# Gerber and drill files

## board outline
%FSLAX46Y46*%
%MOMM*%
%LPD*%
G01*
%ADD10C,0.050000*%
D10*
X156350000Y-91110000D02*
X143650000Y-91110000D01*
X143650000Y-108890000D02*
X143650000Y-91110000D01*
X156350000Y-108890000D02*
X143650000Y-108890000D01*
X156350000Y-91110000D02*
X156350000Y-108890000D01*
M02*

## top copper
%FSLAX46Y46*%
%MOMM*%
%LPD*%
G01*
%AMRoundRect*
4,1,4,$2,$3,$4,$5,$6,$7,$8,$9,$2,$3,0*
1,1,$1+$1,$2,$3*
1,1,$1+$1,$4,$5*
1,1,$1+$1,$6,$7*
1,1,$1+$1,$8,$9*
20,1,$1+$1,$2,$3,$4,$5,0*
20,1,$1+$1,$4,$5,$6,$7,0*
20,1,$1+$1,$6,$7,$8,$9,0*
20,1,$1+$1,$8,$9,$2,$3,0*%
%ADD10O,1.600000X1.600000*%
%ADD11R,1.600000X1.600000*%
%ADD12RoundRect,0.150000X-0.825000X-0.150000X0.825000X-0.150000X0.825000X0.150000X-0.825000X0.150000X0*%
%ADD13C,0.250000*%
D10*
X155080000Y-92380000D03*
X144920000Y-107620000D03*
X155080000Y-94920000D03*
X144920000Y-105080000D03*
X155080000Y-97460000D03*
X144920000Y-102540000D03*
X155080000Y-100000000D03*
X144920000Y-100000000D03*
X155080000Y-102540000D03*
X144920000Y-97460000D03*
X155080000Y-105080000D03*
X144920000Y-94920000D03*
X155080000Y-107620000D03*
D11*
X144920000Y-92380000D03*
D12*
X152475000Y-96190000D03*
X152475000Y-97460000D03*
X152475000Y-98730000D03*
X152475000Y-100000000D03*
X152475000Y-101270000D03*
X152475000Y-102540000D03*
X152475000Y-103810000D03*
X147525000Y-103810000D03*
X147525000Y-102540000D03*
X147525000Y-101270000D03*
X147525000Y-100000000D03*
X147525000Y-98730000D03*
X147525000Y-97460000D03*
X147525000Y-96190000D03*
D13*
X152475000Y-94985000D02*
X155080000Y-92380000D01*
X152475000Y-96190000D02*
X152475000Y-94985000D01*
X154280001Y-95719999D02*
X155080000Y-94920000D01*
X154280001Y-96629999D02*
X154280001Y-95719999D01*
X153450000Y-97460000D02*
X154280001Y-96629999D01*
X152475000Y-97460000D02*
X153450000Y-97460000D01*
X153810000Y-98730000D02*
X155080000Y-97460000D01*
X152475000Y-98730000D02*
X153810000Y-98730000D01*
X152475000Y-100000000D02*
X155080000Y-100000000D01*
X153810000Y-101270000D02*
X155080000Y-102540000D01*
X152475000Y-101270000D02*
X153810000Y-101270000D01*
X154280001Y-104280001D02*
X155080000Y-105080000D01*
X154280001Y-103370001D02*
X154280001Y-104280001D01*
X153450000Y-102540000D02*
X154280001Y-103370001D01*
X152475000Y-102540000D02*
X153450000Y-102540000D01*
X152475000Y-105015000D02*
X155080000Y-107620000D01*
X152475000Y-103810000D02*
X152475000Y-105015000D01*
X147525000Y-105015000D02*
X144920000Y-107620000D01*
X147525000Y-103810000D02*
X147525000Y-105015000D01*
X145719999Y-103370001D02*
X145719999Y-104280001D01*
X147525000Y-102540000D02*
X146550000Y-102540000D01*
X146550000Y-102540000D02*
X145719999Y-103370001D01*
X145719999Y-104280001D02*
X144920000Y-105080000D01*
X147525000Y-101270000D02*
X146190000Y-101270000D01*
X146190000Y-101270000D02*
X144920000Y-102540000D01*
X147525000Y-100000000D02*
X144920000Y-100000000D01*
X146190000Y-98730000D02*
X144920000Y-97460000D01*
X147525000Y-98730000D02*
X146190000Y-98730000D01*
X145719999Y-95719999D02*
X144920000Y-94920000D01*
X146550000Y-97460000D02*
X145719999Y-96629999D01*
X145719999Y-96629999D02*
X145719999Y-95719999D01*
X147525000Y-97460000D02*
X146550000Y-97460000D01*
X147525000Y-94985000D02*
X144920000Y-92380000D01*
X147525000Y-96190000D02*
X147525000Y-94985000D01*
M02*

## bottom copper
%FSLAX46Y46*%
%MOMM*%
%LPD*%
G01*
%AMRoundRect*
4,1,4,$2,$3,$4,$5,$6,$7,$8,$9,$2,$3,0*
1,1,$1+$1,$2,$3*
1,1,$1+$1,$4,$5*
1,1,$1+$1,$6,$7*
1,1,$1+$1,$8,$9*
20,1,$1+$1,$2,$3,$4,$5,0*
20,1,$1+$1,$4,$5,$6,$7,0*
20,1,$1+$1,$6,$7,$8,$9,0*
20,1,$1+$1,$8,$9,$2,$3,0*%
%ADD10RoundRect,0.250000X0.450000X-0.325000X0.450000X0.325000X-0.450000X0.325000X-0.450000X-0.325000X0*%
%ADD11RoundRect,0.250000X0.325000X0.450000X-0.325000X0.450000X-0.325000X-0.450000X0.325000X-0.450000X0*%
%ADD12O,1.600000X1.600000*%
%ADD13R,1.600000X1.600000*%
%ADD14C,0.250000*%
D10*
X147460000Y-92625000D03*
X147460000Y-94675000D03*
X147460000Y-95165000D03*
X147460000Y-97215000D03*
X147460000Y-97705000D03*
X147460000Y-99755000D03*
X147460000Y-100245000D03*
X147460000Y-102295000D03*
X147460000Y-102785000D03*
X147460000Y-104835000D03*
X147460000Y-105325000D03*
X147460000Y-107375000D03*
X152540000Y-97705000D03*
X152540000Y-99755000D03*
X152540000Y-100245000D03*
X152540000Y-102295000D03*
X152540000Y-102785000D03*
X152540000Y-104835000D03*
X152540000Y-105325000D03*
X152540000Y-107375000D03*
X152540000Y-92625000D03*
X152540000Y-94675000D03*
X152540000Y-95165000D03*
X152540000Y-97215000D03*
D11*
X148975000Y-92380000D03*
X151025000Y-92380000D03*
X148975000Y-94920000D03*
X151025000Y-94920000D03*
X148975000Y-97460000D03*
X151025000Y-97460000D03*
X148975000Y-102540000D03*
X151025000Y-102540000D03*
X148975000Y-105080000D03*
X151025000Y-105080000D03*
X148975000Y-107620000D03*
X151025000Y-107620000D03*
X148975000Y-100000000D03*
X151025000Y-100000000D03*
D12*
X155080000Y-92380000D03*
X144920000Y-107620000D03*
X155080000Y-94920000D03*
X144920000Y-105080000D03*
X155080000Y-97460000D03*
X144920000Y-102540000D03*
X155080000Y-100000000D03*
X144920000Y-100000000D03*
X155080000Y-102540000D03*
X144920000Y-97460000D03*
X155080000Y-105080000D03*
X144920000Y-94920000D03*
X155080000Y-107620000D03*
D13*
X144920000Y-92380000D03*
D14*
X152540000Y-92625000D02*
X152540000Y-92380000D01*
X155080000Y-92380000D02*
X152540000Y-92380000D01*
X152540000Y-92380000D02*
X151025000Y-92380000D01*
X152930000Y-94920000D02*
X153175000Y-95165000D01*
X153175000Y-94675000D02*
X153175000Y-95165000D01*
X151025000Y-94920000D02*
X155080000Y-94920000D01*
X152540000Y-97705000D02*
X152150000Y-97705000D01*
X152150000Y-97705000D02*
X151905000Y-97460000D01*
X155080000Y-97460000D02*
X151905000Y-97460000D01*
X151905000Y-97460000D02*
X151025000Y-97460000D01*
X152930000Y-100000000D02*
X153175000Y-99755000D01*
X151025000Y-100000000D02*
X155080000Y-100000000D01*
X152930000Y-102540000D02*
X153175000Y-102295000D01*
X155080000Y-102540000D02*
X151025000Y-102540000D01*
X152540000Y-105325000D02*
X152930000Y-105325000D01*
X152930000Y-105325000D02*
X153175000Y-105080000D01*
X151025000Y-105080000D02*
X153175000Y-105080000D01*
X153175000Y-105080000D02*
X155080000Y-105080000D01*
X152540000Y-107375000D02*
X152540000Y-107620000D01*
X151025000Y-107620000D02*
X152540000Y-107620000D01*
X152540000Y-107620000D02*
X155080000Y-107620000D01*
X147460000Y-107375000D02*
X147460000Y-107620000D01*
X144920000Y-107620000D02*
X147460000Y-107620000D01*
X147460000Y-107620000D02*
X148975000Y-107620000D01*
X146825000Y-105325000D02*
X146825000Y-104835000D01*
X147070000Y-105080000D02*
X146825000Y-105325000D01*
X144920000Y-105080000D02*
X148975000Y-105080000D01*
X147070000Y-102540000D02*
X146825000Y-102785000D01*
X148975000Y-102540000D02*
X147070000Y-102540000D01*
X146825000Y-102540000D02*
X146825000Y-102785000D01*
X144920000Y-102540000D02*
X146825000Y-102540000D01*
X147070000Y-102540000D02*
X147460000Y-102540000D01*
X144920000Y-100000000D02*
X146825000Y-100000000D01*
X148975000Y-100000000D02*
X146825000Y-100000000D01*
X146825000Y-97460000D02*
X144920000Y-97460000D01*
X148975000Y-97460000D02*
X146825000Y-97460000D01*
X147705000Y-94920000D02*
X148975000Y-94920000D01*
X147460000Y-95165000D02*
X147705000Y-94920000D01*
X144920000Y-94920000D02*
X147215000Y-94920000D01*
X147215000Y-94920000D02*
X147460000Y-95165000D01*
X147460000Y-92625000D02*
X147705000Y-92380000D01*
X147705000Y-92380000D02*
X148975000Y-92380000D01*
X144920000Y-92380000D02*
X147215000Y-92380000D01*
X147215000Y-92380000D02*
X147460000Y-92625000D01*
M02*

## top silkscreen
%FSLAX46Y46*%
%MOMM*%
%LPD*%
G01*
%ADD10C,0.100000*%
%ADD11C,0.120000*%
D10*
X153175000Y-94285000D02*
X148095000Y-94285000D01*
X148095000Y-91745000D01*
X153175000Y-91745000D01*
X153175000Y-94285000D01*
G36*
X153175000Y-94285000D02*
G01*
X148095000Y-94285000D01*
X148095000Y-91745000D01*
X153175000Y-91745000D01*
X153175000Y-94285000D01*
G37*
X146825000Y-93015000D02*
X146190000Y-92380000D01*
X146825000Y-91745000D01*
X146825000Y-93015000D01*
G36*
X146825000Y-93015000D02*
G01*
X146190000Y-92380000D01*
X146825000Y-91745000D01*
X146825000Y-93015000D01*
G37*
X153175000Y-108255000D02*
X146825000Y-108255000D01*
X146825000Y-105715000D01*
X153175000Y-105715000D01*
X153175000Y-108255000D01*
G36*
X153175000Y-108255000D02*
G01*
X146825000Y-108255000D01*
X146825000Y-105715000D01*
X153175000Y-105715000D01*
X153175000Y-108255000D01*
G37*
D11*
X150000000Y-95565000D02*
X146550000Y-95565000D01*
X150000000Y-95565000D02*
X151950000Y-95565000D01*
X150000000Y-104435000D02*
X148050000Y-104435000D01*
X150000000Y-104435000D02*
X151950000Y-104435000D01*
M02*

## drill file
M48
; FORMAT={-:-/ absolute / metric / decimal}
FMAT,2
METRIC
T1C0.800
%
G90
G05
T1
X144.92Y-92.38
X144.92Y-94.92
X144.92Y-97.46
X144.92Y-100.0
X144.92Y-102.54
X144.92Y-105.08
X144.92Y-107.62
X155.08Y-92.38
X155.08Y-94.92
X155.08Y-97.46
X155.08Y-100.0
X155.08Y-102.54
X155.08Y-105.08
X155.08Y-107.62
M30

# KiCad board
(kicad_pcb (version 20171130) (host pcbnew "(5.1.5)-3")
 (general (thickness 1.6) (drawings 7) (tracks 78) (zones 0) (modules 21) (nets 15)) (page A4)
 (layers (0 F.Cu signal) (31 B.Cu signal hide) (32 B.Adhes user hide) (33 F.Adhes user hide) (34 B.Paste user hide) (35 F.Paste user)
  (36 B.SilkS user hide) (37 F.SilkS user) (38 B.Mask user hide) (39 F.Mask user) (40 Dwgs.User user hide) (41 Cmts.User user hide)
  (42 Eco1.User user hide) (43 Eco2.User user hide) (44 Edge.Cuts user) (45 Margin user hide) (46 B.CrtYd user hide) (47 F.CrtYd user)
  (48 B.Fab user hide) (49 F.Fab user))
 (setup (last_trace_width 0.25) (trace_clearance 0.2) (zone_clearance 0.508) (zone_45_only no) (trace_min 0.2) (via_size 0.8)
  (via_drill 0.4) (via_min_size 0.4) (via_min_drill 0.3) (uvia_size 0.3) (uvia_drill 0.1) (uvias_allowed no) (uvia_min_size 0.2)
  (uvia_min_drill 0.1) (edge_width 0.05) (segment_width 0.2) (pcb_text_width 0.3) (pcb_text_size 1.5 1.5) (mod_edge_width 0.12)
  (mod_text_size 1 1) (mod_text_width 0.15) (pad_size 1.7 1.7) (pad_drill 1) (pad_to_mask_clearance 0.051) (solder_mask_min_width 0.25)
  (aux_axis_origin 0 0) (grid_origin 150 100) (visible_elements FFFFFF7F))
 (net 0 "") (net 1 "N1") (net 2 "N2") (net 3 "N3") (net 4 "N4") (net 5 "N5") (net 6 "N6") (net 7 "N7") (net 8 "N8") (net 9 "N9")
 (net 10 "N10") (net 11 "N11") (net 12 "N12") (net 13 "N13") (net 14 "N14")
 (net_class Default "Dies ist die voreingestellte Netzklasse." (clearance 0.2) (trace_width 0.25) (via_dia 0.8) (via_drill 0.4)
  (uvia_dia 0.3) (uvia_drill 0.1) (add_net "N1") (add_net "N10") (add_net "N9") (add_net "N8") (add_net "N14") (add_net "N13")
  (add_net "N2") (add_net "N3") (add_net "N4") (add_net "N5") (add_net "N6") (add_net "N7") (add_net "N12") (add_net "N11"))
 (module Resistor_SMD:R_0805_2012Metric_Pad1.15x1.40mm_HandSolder (layer B.Cu) (at 147.46 93.65 90)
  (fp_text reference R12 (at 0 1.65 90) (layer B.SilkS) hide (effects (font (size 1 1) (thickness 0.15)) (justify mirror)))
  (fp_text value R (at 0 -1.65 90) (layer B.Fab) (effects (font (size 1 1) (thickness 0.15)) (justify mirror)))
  (pad 2 smd roundrect (at 1.025 0 90) (size 1.15 1.4) (layers B.Cu B.Paste B.Mask) (roundrect_rratio 0.217391) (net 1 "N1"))
  (pad 1 smd roundrect (at -1.025 0 90) (size 1.15 1.4) (layers B.Cu B.Paste B.Mask) (roundrect_rratio 0.217391) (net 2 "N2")))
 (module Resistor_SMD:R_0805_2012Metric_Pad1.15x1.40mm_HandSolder (layer B.Cu) (at 147.46 96.19 90)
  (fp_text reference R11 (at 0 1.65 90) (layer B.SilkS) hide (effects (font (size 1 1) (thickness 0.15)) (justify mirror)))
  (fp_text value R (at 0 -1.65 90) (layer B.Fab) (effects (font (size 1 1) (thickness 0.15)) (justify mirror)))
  (pad 2 smd roundrect (at 1.025 0 90) (size 1.15 1.4) (layers B.Cu B.Paste B.Mask) (roundrect_rratio 0.217391) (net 2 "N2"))
  (pad 1 smd roundrect (at -1.025 0 90) (size 1.15 1.4) (layers B.Cu B.Paste B.Mask) (roundrect_rratio 0.217391) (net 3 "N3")))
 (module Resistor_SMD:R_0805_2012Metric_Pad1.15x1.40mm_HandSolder (layer B.Cu) (at 147.46 98.73 90)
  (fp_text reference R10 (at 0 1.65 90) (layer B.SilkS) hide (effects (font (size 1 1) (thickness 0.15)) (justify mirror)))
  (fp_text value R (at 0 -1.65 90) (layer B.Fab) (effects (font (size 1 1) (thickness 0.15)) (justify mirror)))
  (pad 2 smd roundrect (at 1.025 0 90) (size 1.15 1.4) (layers B.Cu B.Paste B.Mask) (roundrect_rratio 0.217391) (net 3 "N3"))
  (pad 1 smd roundrect (at -1.025 0 90) (size 1.15 1.4) (layers B.Cu B.Paste B.Mask) (roundrect_rratio 0.217391) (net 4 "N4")))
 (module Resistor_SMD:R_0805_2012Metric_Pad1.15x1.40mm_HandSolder (layer B.Cu) (at 147.46 101.27 90)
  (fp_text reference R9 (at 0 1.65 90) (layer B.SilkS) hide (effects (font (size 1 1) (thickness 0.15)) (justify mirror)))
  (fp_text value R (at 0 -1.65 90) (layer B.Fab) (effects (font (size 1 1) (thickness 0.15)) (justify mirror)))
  (pad 2 smd roundrect (at 1.025 0 90) (size 1.15 1.4) (layers B.Cu B.Paste B.Mask) (roundrect_rratio 0.217391) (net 4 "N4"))
  (pad 1 smd roundrect (at -1.025 0 90) (size 1.15 1.4) (layers B.Cu B.Paste B.Mask) (roundrect_rratio 0.217391) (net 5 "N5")))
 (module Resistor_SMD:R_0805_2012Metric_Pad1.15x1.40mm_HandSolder (layer B.Cu) (at 147.46 103.81 90)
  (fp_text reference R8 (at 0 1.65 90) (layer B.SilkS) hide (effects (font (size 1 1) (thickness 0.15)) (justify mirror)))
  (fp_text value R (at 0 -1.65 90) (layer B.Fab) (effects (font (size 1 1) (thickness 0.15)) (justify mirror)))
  (pad 2 smd roundrect (at 1.025 0 90) (size 1.15 1.4) (layers B.Cu B.Paste B.Mask) (roundrect_rratio 0.217391) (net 5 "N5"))
  (pad 1 smd roundrect (at -1.025 0 90) (size 1.15 1.4) (layers B.Cu B.Paste B.Mask) (roundrect_rratio 0.217391) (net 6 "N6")))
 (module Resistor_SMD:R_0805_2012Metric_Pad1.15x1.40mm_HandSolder (layer B.Cu) (at 147.46 106.35 90)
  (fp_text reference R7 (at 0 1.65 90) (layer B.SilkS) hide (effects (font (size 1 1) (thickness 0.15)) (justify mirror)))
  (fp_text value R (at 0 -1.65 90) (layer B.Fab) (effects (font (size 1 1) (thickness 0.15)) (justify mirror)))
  (pad 2 smd roundrect (at 1.025 0 90) (size 1.15 1.4) (layers B.Cu B.Paste B.Mask) (roundrect_rratio 0.217391) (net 6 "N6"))
  (pad 1 smd roundrect (at -1.025 0 90) (size 1.15 1.4) (layers B.Cu B.Paste B.Mask) (roundrect_rratio 0.217391) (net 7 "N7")))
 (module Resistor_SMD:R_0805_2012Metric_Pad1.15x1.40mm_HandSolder (layer B.Cu) (at 152.54 98.73 90)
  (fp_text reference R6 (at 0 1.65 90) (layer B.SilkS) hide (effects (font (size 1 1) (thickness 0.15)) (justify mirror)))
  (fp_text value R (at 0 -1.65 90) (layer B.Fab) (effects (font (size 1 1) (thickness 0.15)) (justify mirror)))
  (pad 2 smd roundrect (at 1.025 0 90) (size 1.15 1.4) (layers B.Cu B.Paste B.Mask) (roundrect_rratio 0.217391) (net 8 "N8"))
  (pad 1 smd roundrect (at -1.025 0 90) (size 1.15 1.4) (layers B.Cu B.Paste B.Mask) (roundrect_rratio 0.217391) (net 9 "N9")))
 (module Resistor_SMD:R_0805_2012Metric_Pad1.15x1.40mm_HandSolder (layer B.Cu) (at 152.54 101.27 90)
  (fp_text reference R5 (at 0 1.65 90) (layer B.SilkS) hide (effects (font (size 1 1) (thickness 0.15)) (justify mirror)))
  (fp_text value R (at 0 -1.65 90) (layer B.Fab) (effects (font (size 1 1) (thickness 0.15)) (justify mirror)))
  (pad 2 smd roundrect (at 1.025 0 90) (size 1.15 1.4) (layers B.Cu B.Paste B.Mask) (roundrect_rratio 0.217391) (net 9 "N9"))
  (pad 1 smd roundrect (at -1.025 0 90) (size 1.15 1.4) (layers B.Cu B.Paste B.Mask) (roundrect_rratio 0.217391) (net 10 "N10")))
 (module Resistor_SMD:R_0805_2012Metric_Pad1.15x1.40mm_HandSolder (layer B.Cu) (at 152.54 103.81 90)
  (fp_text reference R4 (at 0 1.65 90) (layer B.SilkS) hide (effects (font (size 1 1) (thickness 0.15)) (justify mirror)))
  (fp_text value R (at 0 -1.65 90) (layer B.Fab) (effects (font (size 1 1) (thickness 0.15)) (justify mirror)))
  (pad 2 smd roundrect (at 1.025 0 90) (size 1.15 1.4) (layers B.Cu B.Paste B.Mask) (roundrect_rratio 0.217391) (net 10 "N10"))
  (pad 1 smd roundrect (at -1.025 0 90) (size 1.15 1.4) (layers B.Cu B.Paste B.Mask) (roundrect_rratio 0.217391) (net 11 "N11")))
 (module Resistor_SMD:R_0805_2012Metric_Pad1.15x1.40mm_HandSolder (layer B.Cu) (at 152.54 106.35 90)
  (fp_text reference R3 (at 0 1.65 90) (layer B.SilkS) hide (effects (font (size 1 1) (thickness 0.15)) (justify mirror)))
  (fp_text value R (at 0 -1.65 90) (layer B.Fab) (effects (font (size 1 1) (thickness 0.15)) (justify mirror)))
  (pad 2 smd roundrect (at 1.025 0 90) (size 1.15 1.4) (layers B.Cu B.Paste B.Mask) (roundrect_rratio 0.217391) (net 11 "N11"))
  (pad 1 smd roundrect (at -1.025 0 90) (size 1.15 1.4) (layers B.Cu B.Paste B.Mask) (roundrect_rratio 0.217391) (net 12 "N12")))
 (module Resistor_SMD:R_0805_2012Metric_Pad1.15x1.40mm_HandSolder (layer B.Cu) (at 152.54 93.65 90)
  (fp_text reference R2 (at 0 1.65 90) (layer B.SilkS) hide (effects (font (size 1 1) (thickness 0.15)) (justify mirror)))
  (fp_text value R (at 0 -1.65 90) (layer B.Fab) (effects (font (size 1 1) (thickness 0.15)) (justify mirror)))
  (pad 2 smd roundrect (at 1.025 0 90) (size 1.15 1.4) (layers B.Cu B.Paste B.Mask) (roundrect_rratio 0.217391) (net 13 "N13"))
  (pad 1 smd roundrect (at -1.025 0 90) (size 1.15 1.4) (layers B.Cu B.Paste B.Mask) (roundrect_rratio 0.217391) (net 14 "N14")))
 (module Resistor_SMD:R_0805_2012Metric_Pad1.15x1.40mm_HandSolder (layer B.Cu) (at 152.54 96.19 90)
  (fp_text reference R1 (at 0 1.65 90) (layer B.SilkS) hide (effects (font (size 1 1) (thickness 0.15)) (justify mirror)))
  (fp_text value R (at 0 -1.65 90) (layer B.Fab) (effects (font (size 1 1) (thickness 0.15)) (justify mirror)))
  (pad 2 smd roundrect (at 1.025 0 90) (size 1.15 1.4) (layers B.Cu B.Paste B.Mask) (roundrect_rratio 0.217391) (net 14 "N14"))
  (pad 1 smd roundrect (at -1.025 0 90) (size 1.15 1.4) (layers B.Cu B.Paste B.Mask) (roundrect_rratio 0.217391) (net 8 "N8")))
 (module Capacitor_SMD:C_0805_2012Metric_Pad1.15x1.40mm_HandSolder (layer B.Cu) (at 150 92.38 180)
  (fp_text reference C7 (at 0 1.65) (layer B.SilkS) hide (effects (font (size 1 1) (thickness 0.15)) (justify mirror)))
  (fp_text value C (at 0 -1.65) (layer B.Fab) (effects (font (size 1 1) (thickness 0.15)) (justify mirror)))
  (pad 2 smd roundrect (at 1.025 0 180) (size 1.15 1.4) (layers B.Cu B.Paste B.Mask) (roundrect_rratio 0.217391) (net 1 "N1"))
  (pad 1 smd roundrect (at -1.025 0 180) (size 1.15 1.4) (layers B.Cu B.Paste B.Mask) (roundrect_rratio 0.217391) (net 13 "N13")))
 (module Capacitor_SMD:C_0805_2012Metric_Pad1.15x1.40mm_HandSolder (layer B.Cu) (at 150 94.92 180)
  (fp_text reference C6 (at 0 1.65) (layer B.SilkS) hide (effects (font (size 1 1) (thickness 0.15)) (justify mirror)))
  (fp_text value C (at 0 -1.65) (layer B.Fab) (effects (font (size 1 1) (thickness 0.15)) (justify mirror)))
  (pad 2 smd roundrect (at 1.025 0 180) (size 1.15 1.4) (layers B.Cu B.Paste B.Mask) (roundrect_rratio 0.217391) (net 2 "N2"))
  (pad 1 smd roundrect (at -1.025 0 180) (size 1.15 1.4) (layers B.Cu B.Paste B.Mask) (roundrect_rratio 0.217391) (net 14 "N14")))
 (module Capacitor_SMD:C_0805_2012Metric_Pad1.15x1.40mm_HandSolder (layer B.Cu) (at 150 97.46 180)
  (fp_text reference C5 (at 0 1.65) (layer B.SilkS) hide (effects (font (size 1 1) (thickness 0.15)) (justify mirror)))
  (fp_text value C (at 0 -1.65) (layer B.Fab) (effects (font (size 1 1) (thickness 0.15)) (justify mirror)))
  (pad 2 smd roundrect (at 1.025 0 180) (size 1.15 1.4) (layers B.Cu B.Paste B.Mask) (roundrect_rratio 0.217391) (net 3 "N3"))
  (pad 1 smd roundrect (at -1.025 0 180) (size 1.15 1.4) (layers B.Cu B.Paste B.Mask) (roundrect_rratio 0.217391) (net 8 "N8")))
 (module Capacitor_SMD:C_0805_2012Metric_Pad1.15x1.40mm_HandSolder (layer B.Cu) (at 150 102.54 180)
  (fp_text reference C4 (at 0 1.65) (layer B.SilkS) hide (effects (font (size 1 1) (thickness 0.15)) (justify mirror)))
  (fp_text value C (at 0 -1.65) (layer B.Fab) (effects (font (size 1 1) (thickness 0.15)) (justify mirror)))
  (pad 2 smd roundrect (at 1.025 0 180) (size 1.15 1.4) (layers B.Cu B.Paste B.Mask) (roundrect_rratio 0.217391) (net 5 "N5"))
  (pad 1 smd roundrect (at -1.025 0 180) (size 1.15 1.4) (layers B.Cu B.Paste B.Mask) (roundrect_rratio 0.217391) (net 10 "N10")))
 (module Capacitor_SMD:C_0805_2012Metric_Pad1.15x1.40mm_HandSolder (layer B.Cu) (at 150 105.08 180)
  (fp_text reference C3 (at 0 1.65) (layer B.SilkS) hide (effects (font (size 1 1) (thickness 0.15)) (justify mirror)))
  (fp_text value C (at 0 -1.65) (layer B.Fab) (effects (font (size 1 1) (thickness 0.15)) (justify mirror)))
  (pad 2 smd roundrect (at 1.025 0 180) (size 1.15 1.4) (layers B.Cu B.Paste B.Mask) (roundrect_rratio 0.217391) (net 6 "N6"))
  (pad 1 smd roundrect (at -1.025 0 180) (size 1.15 1.4) (layers B.Cu B.Paste B.Mask) (roundrect_rratio 0.217391) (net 11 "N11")))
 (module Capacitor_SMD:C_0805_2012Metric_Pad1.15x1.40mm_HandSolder (layer B.Cu) (at 150 107.62 180)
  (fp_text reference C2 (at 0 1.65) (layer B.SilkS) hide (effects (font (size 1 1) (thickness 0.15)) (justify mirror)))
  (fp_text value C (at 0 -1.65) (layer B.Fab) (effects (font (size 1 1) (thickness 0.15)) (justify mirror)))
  (pad 2 smd roundrect (at 1.025 0 180) (size 1.15 1.4) (layers B.Cu B.Paste B.Mask) (roundrect_rratio 0.217391) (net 7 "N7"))
  (pad 1 smd roundrect (at -1.025 0 180) (size 1.15 1.4) (layers B.Cu B.Paste B.Mask) (roundrect_rratio 0.217391) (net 12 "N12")))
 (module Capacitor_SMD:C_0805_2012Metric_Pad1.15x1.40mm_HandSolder (layer B.Cu) (at 150 100 180)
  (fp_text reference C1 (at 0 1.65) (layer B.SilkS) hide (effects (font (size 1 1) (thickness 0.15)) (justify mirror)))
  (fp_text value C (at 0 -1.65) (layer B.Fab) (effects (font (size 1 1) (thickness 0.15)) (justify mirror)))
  (pad 2 smd roundrect (at 1.025 0 180) (size 1.15 1.4) (layers B.Cu B.Paste B.Mask) (roundrect_rratio 0.217391) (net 4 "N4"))
  (pad 1 smd roundrect (at -1.025 0 180) (size 1.15 1.4) (layers B.Cu B.Paste B.Mask) (roundrect_rratio 0.217391) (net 9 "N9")))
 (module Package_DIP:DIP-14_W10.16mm (layer F.Cu) (at 150 100)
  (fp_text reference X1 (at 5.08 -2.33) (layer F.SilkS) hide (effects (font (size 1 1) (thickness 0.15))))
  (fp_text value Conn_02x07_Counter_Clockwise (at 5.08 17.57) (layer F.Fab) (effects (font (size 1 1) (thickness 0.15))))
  (pad 14 thru_hole oval (at 5.08 -7.62) (size 1.6 1.6) (drill 0.8) (layers *.Cu *.Mask) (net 13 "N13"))
  (pad 7 thru_hole oval (at -5.08 7.62) (size 1.6 1.6) (drill 0.8) (layers *.Cu *.Mask) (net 7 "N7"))
  (pad 13 thru_hole oval (at 5.08 -5.08) (size 1.6 1.6) (drill 0.8) (layers *.Cu *.Mask) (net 14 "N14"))
  (pad 6 thru_hole oval (at -5.08 5.08) (size 1.6 1.6) (drill 0.8) (layers *.Cu *.Mask) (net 6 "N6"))
  (pad 12 thru_hole oval (at 5.08 -2.54) (size 1.6 1.6) (drill 0.8) (layers *.Cu *.Mask) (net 8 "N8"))
  (pad 5 thru_hole oval (at -5.08 2.54) (size 1.6 1.6) (drill 0.8) (layers *.Cu *.Mask) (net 5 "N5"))
  (pad 11 thru_hole oval (at 5.08 0) (size 1.6 1.6) (drill 0.8) (layers *.Cu *.Mask) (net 9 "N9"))
  (pad 4 thru_hole oval (at -5.08 0) (size 1.6 1.6) (drill 0.8) (layers *.Cu *.Mask) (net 4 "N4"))
  (pad 10 thru_hole oval (at 5.08 2.54) (size 1.6 1.6) (drill 0.8) (layers *.Cu *.Mask) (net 10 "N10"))
  (pad 3 thru_hole oval (at -5.08 -2.54) (size 1.6 1.6) (drill 0.8) (layers *.Cu *.Mask) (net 3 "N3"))
  (pad 9 thru_hole oval (at 5.08 5.08) (size 1.6 1.6) (drill 0.8) (layers *.Cu *.Mask) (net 11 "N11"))
  (pad 2 thru_hole oval (at -5.08 -5.08) (size 1.6 1.6) (drill 0.8) (layers *.Cu *.Mask) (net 2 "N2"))
  (pad 8 thru_hole oval (at 5.08 7.62) (size 1.6 1.6) (drill 0.8) (layers *.Cu *.Mask) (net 12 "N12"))
  (pad 1 thru_hole rect (at -5.08 -7.62) (size 1.6 1.6) (drill 0.8) (layers *.Cu *.Mask) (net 1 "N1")))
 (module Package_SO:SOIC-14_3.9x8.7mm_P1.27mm (layer F.Cu) (at 150 100)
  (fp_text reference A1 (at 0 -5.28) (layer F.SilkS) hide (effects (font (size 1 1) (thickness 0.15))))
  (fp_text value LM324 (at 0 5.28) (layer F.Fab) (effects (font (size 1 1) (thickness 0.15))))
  (fp_line (start 0 -4.435) (end -3.45 -4.435) (layer F.SilkS) (width 0.12))
  (fp_line (start 0 -4.435) (end 1.95 -4.435) (layer F.SilkS) (width 0.12))
  (fp_line (start 0 4.435) (end -1.95 4.435) (layer F.SilkS) (width 0.12))
  (fp_line (start 0 4.435) (end 1.95 4.435) (layer F.SilkS) (width 0.12))
  (pad 14 smd roundrect (at 2.475 -3.81) (size 1.95 0.6) (layers F.Cu F.Paste F.Mask) (roundrect_rratio 0.25) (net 13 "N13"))
  (pad 13 smd roundrect (at 2.475 -2.54) (size 1.95 0.6) (layers F.Cu F.Paste F.Mask) (roundrect_rratio 0.25) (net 14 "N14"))
  (pad 12 smd roundrect (at 2.475 -1.27) (size 1.95 0.6) (layers F.Cu F.Paste F.Mask) (roundrect_rratio 0.25) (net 8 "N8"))
  (pad 11 smd roundrect (at 2.475 0) (size 1.95 0.6) (layers F.Cu F.Paste F.Mask) (roundrect_rratio 0.25) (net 9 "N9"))
  (pad 10 smd roundrect (at 2.475 1.27) (size 1.95 0.6) (layers F.Cu F.Paste F.Mask) (roundrect_rratio 0.25) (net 10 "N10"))
  (pad 9 smd roundrect (at 2.475 2.54) (size 1.95 0.6) (layers F.Cu F.Paste F.Mask) (roundrect_rratio 0.25) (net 11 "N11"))
  (pad 8 smd roundrect (at 2.475 3.81) (size 1.95 0.6) (layers F.Cu F.Paste F.Mask) (roundrect_rratio 0.25) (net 12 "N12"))
  (pad 7 smd roundrect (at -2.475 3.81) (size 1.95 0.6) (layers F.Cu F.Paste F.Mask) (roundrect_rratio 0.25) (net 7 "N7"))
  (pad 6 smd roundrect (at -2.475 2.54) (size 1.95 0.6) (layers F.Cu F.Paste F.Mask) (roundrect_rratio 0.25) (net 6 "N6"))
  (pad 5 smd roundrect (at -2.475 1.27) (size 1.95 0.6) (layers F.Cu F.Paste F.Mask) (roundrect_rratio 0.25) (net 5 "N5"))
  (pad 4 smd roundrect (at -2.475 0) (size 1.95 0.6) (layers F.Cu F.Paste F.Mask) (roundrect_rratio 0.25) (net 4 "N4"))
  (pad 3 smd roundrect (at -2.475 -1.27) (size 1.95 0.6) (layers F.Cu F.Paste F.Mask) (roundrect_rratio 0.25) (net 3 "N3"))
  (pad 2 smd roundrect (at -2.475 -2.54) (size 1.95 0.6) (layers F.Cu F.Paste F.Mask) (roundrect_rratio 0.25) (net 2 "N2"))
  (pad 1 smd roundrect (at -2.475 -3.81) (size 1.95 0.6) (layers F.Cu F.Paste F.Mask) (roundrect_rratio 0.25) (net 1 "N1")))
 (gr_poly (pts (xy 153.175 94.285) (xy 148.095 94.285) (xy 148.095 91.745) (xy 153.175 91.745)) (layer F.SilkS) (width 0.1))
 (gr_poly (pts (xy 146.825 93.015) (xy 146.19 92.38) (xy 146.825 91.745)) (layer F.SilkS) (width 0.1))
 (gr_poly (pts (xy 153.175 108.255) (xy 146.825 108.255) (xy 146.825 105.715) (xy 153.175 105.715)) (layer F.SilkS) (width 0.1))
 (gr_line (start 156.35 91.11) (end 143.65 91.11) (layer Edge.Cuts) (width 0.05))
 (gr_line (start 143.65 108.89) (end 143.65 91.11) (layer Edge.Cuts) (width 0.05))
 (gr_line (start 156.35 108.89) (end 143.65 108.89) (layer Edge.Cuts) (width 0.05))
 (gr_line (start 156.35 91.11) (end 156.35 108.89) (layer Edge.Cuts) (width 0.05))
 (segment (start 152.475 94.985) (end 155.08 92.38) (width 0.25) (layer F.Cu) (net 13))
 (segment (start 152.475 96.19) (end 152.475 94.985) (width 0.25) (layer F.Cu) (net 13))
 (segment (start 152.54 92.625) (end 152.54 92.38) (width 0.25) (layer B.Cu) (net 13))
 (segment (start 155.08 92.38) (end 152.54 92.38) (width 0.25) (layer B.Cu) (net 13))
 (segment (start 152.54 92.38) (end 151.025 92.38) (width 0.25) (layer B.Cu) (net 13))
 (segment (start 154.280001 95.719999) (end 155.08 94.92) (width 0.25) (layer F.Cu) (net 14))
 (segment (start 154.280001 96.629999) (end 154.280001 95.719999) (width 0.25) (layer F.Cu) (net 14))
 (segment (start 153.45 97.46) (end 154.280001 96.629999) (width 0.25) (layer F.Cu) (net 14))
 (segment (start 152.475 97.46) (end 153.45 97.46) (width 0.25) (layer F.Cu) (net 14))
 (segment (start 152.93 94.92) (end 153.175 95.165) (width 0.25) (layer B.Cu) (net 14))
 (segment (start 153.175 94.675) (end 153.175 95.165) (width 0.25) (layer B.Cu) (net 14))
 (segment (start 151.025 94.92) (end 155.08 94.92) (width 0.25) (layer B.Cu) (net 14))
 (segment (start 153.81 98.73) (end 155.08 97.46) (width 0.25) (layer F.Cu) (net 8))
 (segment (start 152.475 98.73) (end 153.81 98.73) (width 0.25) (layer F.Cu) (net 8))
 (segment (start 152.54 97.705) (end 152.15 97.705) (width 0.25) (layer B.Cu) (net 8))
 (segment (start 152.15 97.705) (end 151.905 97.46) (width 0.25) (layer B.Cu) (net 8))
 (segment (start 155.08 97.46) (end 151.905 97.46) (width 0.25) (layer B.Cu) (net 8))
 (segment (start 151.905 97.46) (end 151.025 97.46) (width 0.25) (layer B.Cu) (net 8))
 (segment (start 152.475 100) (end 155.08 100) (width 0.25) (layer F.Cu) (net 9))
 (segment (start 152.93 100) (end 153.175 99.755) (width 0.25) (layer B.Cu) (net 9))
 (segment (start 151.025 100) (end 155.08 100) (width 0.25) (layer B.Cu) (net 9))
 (segment (start 153.81 101.27) (end 155.08 102.54) (width 0.25) (layer F.Cu) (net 10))
 (segment (start 152.475 101.27) (end 153.81 101.27) (width 0.25) (layer F.Cu) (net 10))
 (segment (start 152.93 102.54) (end 153.175 102.295) (width 0.25) (layer B.Cu) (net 10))
 (segment (start 155.08 102.54) (end 151.025 102.54) (width 0.25) (layer B.Cu) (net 10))
 (segment (start 154.280001 104.280001) (end 155.08 105.08) (width 0.25) (layer F.Cu) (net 11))
 (segment (start 154.280001 103.370001) (end 154.280001 104.280001) (width 0.25) (layer F.Cu) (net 11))
 (segment (start 153.45 102.54) (end 154.280001 103.370001) (width 0.25) (layer F.Cu) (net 11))
 (segment (start 152.475 102.54) (end 153.45 102.54) (width 0.25) (layer F.Cu) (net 11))
 (segment (start 152.54 105.325) (end 152.93 105.325) (width 0.25) (layer B.Cu) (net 11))
 (segment (start 152.93 105.325) (end 153.175 105.08) (width 0.25) (layer B.Cu) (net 11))
 (segment (start 151.025 105.08) (end 153.175 105.08) (width 0.25) (layer B.Cu) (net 11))
 (segment (start 153.175 105.08) (end 155.08 105.08) (width 0.25) (layer B.Cu) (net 11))
 (segment (start 152.475 105.015) (end 155.08 107.62) (width 0.25) (layer F.Cu) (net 12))
 (segment (start 152.475 103.81) (end 152.475 105.015) (width 0.25) (layer F.Cu) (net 12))
 (segment (start 152.54 107.375) (end 152.54 107.62) (width 0.25) (layer B.Cu) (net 12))
 (segment (start 151.025 107.62) (end 152.54 107.62) (width 0.25) (layer B.Cu) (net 12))
 (segment (start 152.54 107.62) (end 155.08 107.62) (width 0.25) (layer B.Cu) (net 12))
 (segment (start 147.525 105.015) (end 144.92 107.62) (width 0.25) (layer F.Cu) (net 7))
 (segment (start 147.525 103.81) (end 147.525 105.015) (width 0.25) (layer F.Cu) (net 7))
 (segment (start 147.46 107.375) (end 147.46 107.62) (width 0.25) (layer B.Cu) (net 7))
 (segment (start 144.92 107.62) (end 147.46 107.62) (width 0.25) (layer B.Cu) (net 7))
 (segment (start 147.46 107.62) (end 148.975 107.62) (width 0.25) (layer B.Cu) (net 7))
 (segment (start 145.719999 103.370001) (end 145.719999 104.280001) (width 0.25) (layer F.Cu) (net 6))
 (segment (start 147.525 102.54) (end 146.55 102.54) (width 0.25) (layer F.Cu) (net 6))
 (segment (start 146.55 102.54) (end 145.719999 103.370001) (width 0.25) (layer F.Cu) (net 6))
 (segment (start 145.719999 104.280001) (end 144.92 105.08) (width 0.25) (layer F.Cu) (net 6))
 (segment (start 146.825 105.325) (end 146.825 104.835) (width 0.25) (layer B.Cu) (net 6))
 (segment (start 147.07 105.08) (end 146.825 105.325) (width 0.25) (layer B.Cu) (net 6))
 (segment (start 144.92 105.08) (end 148.975 105.08) (width 0.25) (layer B.Cu) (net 6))
 (segment (start 147.525 101.27) (end 146.19 101.27) (width 0.25) (layer F.Cu) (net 5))
 (segment (start 146.19 101.27) (end 144.92 102.54) (width 0.25) (layer F.Cu) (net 5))
 (segment (start 147.07 102.54) (end 146.825 102.785) (width 0.25) (layer B.Cu) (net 5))
 (segment (start 148.975 102.54) (end 147.07 102.54) (width 0.25) (layer B.Cu) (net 5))
 (segment (start 146.825 102.54) (end 146.825 102.785) (width 0.25) (layer B.Cu) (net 5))
 (segment (start 144.92 102.54) (end 146.825 102.54) (width 0.25) (layer B.Cu) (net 5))
 (segment (start 147.07 102.54) (end 147.46 102.54) (width 0.25) (layer B.Cu) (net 5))
 (segment (start 147.525 100) (end 144.92 100) (width 0.25) (layer F.Cu) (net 4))
 (segment (start 144.92 100) (end 146.825 100) (width 0.25) (layer B.Cu) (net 4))
 (segment (start 148.975 100) (end 146.825 100) (width 0.25) (layer B.Cu) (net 4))
 (segment (start 146.19 98.73) (end 144.92 97.46) (width 0.25) (layer F.Cu) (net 3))
 (segment (start 147.525 98.73) (end 146.19 98.73) (width 0.25) (layer F.Cu) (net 3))
 (segment (start 146.825 97.46) (end 144.92 97.46) (width 0.25) (layer B.Cu) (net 3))
 (segment (start 148.975 97.46) (end 146.825 97.46) (width 0.25) (layer B.Cu) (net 3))
 (segment (start 145.719999 95.719999) (end 144.92 94.92) (width 0.25) (layer F.Cu) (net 2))
 (segment (start 146.55 97.46) (end 145.719999 96.629999) (width 0.25) (layer F.Cu) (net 2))
 (segment (start 145.719999 96.629999) (end 145.719999 95.719999) (width 0.25) (layer F.Cu) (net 2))
 (segment (start 147.525 97.46) (end 146.55 97.46) (width 0.25) (layer F.Cu) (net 2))
 (segment (start 147.705 94.92) (end 148.975 94.92) (width 0.25) (layer B.Cu) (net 2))
 (segment (start 147.46 95.165) (end 147.705 94.92) (width 0.25) (layer B.Cu) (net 2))
 (segment (start 144.92 94.92) (end 147.215 94.92) (width 0.25) (layer B.Cu) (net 2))
 (segment (start 147.215 94.92) (end 147.46 95.165) (width 0.25) (layer B.Cu) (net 2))
 (segment (start 147.525 94.985) (end 144.92 92.38) (width 0.25) (layer F.Cu) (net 1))
 (segment (start 147.525 96.19) (end 147.525 94.985) (width 0.25) (layer F.Cu) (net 1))
 (segment (start 147.46 92.625) (end 147.705 92.38) (width 0.25) (layer B.Cu) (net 1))
 (segment (start 147.705 92.38) (end 148.975 92.38) (width 0.25) (layer B.Cu) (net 1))
 (segment (start 144.92 92.38) (end 147.215 92.38) (width 0.25) (layer B.Cu) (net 1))
 (segment (start 147.215 92.38) (end 147.46 92.625) (width 0.25) (layer B.Cu) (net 1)))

